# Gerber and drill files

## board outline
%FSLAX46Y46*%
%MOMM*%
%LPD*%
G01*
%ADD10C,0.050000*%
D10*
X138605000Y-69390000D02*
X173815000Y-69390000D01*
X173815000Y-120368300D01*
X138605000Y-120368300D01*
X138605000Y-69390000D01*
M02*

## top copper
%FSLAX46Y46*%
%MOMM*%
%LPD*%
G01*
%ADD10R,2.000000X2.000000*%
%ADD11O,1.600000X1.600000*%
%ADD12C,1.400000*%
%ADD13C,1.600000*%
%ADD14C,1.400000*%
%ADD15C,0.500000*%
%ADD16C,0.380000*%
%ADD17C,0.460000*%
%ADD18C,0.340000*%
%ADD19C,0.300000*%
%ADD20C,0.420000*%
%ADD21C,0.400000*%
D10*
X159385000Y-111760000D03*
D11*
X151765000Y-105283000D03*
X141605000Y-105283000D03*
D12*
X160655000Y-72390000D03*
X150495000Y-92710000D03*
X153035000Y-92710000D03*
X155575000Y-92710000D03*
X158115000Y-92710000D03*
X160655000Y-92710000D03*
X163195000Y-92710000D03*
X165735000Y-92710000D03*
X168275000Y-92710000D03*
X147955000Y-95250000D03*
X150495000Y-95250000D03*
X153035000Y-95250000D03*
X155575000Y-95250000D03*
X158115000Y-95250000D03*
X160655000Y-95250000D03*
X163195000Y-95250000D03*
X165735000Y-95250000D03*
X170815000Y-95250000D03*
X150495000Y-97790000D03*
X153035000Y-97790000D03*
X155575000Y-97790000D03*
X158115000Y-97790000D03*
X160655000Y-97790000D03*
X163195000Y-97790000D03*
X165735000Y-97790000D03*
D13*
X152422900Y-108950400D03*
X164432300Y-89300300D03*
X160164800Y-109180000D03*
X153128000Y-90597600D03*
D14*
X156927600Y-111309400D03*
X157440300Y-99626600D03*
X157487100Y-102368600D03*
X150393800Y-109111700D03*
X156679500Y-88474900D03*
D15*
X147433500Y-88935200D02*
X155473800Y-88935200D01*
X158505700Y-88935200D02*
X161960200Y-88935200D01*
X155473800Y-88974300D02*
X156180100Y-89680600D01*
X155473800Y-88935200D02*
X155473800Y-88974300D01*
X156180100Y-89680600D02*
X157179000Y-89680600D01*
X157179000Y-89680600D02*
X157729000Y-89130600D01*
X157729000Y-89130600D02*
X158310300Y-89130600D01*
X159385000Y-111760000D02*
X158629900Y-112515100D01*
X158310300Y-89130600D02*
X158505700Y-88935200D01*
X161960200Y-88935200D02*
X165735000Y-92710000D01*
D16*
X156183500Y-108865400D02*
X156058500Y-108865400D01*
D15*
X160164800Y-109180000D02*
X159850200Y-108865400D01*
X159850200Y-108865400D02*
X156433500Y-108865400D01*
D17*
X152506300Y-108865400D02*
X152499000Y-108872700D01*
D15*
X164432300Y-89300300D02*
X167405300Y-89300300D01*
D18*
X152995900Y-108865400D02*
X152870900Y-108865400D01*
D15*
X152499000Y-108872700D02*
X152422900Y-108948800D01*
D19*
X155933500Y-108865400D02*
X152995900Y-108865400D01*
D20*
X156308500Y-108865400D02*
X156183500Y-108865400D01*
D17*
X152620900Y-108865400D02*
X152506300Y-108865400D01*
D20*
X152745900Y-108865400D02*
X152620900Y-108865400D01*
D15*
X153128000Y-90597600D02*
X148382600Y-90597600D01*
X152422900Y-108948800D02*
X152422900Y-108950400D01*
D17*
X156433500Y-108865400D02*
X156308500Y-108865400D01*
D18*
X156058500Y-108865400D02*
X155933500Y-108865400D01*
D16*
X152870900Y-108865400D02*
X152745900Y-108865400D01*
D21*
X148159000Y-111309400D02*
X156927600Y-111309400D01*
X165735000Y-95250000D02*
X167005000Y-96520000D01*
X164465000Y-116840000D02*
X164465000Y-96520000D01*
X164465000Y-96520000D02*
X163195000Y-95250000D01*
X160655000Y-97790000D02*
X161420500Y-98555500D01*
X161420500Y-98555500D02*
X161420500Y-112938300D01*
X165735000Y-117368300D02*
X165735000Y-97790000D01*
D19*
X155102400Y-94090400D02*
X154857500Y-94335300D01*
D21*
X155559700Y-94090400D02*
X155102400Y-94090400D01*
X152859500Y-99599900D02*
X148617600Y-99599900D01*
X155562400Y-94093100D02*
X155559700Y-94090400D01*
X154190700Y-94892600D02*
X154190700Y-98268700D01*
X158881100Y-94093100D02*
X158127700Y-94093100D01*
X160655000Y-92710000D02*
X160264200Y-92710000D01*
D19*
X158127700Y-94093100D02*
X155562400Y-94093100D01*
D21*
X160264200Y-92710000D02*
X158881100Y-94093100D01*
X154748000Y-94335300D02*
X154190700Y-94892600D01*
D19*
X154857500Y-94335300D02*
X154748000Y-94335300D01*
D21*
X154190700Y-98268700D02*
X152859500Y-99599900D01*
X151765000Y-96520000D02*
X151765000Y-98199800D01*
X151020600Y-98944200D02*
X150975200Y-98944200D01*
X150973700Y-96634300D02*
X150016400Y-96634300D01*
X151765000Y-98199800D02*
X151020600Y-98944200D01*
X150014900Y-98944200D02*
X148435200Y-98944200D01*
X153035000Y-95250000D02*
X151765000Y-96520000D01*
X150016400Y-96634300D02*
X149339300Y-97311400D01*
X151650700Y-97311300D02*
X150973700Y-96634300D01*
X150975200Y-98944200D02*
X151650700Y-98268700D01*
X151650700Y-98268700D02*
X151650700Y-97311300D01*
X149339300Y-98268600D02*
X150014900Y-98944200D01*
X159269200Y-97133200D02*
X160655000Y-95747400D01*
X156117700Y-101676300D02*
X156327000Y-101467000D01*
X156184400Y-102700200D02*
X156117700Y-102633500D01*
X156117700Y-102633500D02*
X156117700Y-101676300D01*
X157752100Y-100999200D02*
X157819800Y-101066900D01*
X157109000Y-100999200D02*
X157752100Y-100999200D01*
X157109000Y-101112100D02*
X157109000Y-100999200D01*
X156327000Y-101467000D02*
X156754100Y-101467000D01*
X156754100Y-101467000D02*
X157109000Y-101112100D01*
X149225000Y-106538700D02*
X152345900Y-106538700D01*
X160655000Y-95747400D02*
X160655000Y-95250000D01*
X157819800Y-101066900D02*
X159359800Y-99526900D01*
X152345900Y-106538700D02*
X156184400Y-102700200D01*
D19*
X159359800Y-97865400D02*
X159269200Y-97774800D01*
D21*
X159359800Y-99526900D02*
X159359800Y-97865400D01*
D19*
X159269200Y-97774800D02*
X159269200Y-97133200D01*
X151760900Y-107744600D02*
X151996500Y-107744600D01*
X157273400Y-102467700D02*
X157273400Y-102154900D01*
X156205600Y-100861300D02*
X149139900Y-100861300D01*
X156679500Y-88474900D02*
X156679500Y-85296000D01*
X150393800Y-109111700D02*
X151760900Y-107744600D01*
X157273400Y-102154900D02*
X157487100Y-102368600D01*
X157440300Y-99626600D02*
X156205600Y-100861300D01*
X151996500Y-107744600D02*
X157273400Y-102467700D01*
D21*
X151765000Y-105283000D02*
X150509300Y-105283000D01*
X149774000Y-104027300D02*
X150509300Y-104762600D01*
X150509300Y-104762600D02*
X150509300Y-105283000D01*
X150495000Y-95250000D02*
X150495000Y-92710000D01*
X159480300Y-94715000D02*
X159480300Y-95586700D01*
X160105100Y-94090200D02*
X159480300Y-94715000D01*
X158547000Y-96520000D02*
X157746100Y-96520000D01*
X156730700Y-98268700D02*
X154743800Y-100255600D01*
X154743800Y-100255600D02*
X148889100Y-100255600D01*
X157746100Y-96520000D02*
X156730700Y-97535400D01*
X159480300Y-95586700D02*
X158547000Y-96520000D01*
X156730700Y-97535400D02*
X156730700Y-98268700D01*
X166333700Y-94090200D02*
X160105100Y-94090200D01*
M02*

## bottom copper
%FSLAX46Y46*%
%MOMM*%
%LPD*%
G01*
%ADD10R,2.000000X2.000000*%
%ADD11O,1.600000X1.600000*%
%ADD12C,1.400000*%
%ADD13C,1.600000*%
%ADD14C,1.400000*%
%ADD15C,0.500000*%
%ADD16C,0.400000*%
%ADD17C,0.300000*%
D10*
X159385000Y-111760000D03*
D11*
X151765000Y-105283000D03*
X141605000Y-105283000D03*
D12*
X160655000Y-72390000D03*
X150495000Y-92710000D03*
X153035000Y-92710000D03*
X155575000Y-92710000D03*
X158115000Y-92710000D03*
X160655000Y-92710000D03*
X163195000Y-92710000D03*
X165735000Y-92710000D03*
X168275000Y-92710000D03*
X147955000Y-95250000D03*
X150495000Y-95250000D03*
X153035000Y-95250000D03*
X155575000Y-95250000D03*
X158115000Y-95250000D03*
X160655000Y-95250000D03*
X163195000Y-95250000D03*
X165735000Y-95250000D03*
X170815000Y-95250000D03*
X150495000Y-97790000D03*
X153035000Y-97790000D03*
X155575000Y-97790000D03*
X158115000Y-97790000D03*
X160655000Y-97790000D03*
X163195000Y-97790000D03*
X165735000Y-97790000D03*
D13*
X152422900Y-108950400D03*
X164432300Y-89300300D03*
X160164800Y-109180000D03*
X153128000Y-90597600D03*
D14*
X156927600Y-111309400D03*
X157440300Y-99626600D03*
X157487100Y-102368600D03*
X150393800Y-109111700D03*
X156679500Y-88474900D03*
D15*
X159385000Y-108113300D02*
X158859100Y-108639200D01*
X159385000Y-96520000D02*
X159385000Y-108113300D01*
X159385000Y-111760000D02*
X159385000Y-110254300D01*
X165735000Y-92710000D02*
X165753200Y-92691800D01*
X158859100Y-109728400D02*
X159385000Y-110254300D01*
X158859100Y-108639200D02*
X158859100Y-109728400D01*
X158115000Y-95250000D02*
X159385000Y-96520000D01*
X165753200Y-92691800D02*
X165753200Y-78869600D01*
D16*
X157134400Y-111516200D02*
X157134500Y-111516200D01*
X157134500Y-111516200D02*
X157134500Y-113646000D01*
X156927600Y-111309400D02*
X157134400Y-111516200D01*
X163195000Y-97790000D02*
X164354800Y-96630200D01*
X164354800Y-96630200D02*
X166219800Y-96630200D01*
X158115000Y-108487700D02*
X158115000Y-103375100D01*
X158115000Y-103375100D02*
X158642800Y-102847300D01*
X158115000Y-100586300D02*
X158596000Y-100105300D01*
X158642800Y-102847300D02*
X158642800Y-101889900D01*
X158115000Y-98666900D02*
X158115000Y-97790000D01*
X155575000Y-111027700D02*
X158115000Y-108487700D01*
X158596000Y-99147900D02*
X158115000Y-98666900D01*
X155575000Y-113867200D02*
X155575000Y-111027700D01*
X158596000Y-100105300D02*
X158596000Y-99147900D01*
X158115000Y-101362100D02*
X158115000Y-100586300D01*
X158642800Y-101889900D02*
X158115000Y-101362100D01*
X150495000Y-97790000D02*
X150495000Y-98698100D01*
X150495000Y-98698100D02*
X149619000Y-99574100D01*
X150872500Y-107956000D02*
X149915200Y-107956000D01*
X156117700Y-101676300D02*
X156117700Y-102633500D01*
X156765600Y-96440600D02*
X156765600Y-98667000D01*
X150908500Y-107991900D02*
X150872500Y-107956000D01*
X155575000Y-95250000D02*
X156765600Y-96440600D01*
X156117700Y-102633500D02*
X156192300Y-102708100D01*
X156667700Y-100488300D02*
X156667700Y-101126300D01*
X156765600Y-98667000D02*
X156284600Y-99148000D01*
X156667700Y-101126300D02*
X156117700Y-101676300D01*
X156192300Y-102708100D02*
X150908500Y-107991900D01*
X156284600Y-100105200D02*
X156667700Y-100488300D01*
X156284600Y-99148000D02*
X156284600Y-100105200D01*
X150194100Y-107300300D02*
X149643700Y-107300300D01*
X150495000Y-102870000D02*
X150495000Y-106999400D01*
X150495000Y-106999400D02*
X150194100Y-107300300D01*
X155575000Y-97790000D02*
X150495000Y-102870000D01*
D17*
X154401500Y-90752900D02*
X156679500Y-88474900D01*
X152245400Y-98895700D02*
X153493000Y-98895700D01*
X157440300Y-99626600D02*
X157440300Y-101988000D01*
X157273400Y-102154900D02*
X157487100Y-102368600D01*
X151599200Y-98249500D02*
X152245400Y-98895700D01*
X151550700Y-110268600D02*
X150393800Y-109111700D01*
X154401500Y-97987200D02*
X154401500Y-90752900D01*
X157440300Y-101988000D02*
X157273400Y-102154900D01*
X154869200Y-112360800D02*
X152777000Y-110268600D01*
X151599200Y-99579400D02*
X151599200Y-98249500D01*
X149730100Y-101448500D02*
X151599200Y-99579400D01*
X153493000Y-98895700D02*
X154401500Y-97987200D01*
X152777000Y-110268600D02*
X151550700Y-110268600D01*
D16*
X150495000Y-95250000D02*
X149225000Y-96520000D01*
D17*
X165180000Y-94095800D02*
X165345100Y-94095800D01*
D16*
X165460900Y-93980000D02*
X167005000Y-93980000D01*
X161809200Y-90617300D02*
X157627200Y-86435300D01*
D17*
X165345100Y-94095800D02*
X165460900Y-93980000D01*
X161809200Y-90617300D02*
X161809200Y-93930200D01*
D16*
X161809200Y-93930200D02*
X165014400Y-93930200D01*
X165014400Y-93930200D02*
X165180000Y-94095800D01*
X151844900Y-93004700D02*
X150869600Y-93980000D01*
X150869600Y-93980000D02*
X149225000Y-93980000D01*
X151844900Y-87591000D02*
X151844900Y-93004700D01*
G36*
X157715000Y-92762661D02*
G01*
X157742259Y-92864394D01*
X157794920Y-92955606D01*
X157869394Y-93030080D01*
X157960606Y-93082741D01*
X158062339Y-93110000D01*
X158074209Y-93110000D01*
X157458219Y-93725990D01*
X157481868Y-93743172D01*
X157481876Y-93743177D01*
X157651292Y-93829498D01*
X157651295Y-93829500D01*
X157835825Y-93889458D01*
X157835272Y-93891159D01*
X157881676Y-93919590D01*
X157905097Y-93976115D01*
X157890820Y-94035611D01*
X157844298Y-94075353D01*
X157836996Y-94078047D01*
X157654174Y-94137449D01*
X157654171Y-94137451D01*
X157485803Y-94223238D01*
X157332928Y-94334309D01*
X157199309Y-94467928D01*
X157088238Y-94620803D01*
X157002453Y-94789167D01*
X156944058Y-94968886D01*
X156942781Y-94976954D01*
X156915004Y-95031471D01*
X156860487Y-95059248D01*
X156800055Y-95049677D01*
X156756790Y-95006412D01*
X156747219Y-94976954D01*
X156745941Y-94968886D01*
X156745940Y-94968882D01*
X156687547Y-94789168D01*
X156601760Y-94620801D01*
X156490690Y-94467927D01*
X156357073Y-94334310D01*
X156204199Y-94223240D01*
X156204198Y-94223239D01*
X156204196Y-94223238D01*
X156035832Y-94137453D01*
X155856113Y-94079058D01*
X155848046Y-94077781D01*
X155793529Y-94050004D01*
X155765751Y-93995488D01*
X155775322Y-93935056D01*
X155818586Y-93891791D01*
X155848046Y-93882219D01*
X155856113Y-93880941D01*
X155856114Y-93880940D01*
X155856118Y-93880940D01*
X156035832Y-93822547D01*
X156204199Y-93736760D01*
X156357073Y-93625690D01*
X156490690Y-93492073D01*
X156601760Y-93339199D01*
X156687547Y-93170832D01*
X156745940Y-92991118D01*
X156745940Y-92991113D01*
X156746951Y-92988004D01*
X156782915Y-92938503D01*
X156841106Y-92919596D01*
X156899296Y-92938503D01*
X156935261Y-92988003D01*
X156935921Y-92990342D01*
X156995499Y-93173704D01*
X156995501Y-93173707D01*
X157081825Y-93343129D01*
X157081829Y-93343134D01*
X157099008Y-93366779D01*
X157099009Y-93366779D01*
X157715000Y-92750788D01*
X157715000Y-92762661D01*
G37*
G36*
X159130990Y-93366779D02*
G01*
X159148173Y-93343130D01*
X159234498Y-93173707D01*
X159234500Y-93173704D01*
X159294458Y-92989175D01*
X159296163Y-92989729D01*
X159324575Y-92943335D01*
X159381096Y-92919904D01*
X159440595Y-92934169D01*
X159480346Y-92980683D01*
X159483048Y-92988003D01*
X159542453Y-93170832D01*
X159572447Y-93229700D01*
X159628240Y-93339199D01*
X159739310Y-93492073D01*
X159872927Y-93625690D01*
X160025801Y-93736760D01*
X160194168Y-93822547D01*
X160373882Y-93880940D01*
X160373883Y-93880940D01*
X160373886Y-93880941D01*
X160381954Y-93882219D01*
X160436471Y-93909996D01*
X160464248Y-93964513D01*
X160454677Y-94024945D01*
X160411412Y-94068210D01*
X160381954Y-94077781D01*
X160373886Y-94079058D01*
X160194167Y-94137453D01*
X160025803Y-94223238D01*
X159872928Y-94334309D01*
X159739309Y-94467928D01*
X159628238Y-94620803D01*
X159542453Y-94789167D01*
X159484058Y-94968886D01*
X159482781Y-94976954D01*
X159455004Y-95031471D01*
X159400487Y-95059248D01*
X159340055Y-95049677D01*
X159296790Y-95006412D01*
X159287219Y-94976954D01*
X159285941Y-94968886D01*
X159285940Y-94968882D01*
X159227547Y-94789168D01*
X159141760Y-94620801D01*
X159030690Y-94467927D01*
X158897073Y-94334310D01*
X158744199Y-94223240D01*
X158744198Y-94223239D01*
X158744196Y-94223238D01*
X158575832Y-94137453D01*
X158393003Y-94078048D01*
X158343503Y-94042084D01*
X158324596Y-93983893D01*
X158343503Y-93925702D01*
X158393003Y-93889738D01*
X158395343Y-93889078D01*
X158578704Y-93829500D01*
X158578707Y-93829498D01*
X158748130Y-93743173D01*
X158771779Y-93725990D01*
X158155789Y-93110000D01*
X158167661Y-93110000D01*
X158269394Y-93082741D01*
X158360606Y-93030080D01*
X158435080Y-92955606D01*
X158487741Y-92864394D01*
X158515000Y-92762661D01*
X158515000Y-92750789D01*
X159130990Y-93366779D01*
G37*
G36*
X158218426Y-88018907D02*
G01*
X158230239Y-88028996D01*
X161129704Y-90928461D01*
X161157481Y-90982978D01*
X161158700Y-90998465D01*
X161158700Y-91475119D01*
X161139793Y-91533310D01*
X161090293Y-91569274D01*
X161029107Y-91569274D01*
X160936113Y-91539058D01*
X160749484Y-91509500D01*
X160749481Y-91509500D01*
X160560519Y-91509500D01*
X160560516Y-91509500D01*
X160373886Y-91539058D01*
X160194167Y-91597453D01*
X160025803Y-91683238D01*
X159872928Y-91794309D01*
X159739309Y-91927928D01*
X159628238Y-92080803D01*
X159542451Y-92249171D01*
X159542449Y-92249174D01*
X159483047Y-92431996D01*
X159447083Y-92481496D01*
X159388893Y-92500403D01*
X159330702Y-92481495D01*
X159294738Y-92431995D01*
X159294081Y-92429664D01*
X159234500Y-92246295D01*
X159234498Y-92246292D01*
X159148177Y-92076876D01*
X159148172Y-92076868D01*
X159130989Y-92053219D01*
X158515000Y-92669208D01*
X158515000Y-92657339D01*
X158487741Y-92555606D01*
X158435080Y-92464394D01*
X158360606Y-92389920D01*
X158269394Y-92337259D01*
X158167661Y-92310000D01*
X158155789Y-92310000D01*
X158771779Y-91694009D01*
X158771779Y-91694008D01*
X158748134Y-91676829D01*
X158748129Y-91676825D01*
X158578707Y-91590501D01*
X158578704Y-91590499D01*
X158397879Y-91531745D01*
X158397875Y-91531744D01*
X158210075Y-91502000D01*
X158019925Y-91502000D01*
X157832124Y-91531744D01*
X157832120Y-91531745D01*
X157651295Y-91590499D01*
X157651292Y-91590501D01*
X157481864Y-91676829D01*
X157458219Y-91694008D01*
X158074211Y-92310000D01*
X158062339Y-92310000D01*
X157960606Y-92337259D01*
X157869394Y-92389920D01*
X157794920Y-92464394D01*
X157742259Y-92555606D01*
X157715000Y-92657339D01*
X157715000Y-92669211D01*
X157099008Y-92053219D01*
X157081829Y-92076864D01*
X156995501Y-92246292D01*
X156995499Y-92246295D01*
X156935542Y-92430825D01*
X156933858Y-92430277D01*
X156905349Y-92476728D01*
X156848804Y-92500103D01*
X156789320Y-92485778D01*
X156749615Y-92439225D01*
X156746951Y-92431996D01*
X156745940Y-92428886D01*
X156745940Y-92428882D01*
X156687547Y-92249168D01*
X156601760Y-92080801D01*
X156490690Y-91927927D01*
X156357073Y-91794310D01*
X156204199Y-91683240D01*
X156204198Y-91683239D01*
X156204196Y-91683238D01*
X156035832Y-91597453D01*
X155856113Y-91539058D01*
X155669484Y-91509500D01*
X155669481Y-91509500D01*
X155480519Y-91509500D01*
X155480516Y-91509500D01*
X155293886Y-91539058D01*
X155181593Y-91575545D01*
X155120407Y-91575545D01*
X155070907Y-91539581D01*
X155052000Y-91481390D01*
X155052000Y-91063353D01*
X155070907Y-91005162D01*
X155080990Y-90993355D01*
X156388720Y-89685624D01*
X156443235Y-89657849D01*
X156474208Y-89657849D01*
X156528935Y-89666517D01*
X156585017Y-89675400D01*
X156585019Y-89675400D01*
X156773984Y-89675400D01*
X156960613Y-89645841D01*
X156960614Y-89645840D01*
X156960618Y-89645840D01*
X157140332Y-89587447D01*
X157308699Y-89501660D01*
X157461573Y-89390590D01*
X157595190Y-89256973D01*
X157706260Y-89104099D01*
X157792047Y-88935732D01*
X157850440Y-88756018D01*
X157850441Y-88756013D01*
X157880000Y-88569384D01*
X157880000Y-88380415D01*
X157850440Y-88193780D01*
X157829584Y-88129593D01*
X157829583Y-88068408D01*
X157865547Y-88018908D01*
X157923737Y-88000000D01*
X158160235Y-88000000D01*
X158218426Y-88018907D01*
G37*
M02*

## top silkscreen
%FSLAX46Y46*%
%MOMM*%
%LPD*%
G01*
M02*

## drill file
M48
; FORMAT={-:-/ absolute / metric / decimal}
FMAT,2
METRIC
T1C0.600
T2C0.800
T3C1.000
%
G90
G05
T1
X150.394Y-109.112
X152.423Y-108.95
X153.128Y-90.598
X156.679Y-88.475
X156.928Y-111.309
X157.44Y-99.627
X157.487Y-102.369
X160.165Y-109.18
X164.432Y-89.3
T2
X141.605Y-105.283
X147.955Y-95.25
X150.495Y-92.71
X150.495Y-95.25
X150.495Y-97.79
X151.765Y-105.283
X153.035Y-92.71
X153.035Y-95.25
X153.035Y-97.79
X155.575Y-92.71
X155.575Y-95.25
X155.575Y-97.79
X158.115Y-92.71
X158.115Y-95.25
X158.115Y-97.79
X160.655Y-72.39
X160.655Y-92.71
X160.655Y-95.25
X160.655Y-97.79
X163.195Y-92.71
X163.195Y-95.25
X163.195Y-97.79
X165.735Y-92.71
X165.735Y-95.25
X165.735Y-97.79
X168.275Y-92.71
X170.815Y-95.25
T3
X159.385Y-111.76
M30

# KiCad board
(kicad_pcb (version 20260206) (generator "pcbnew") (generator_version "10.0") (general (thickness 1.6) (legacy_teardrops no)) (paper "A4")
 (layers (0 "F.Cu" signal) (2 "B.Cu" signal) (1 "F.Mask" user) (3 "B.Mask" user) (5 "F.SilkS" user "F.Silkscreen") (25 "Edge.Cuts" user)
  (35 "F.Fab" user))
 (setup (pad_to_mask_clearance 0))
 (gr_rect (start 138.605 69.39) (end 173.815 120.3683) (stroke (width 0.05) (type default)) (fill no) (layer "Edge.Cuts"))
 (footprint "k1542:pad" (layer "F.Cu") (at 159.385 111.76 0.0)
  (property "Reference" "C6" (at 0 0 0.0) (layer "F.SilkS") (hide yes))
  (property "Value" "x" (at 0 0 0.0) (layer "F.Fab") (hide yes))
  (pad "1" thru_hole rect (at 0 0 0.0) (size 2.0 2.0) (drill 1.0) (layers "*.Cu" "*.Mask") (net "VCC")))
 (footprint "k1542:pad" (layer "F.Cu") (at 151.765 105.283 90.0)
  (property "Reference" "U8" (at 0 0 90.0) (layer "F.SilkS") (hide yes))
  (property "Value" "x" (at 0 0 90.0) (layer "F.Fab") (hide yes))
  (pad "13" thru_hole oval (at 0 0 90.0) (size 1.6 1.6) (drill 0.8) (layers "*.Cu" "*.Mask") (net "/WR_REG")))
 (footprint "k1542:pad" (layer "F.Cu") (at 141.605 105.283 90.0)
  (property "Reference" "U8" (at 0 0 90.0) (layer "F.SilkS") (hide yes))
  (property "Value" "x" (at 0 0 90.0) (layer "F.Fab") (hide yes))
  (pad "17" thru_hole oval (at 0 0 90.0) (size 1.6 1.6) (drill 0.8) (layers "*.Cu" "*.Mask") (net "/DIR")))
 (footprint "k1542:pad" (layer "F.Cu") (at 160.655 72.39 180.0)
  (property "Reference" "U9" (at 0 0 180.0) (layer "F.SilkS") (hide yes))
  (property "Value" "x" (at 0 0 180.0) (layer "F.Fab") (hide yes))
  (pad "C8" thru_hole circle (at 0 0 180.0) (size 1.4 1.4) (drill 0.8) (layers "*.Cu" "*.Mask") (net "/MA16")))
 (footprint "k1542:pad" (layer "F.Cu") (at 150.495 92.71 180.0)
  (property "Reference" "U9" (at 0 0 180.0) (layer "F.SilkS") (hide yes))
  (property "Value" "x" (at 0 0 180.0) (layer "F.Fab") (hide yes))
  (pad "L4" thru_hole circle (at 0 0 180.0) (size 1.4 1.4) (drill 0.8) (layers "*.Cu" "*.Mask") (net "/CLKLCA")))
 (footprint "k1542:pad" (layer "F.Cu") (at 153.035 92.71 180.0)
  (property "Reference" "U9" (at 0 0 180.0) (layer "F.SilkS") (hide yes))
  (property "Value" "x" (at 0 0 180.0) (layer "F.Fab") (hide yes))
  (pad "L5" thru_hole circle (at 0 0 180.0) (size 1.4 1.4) (drill 0.8) (layers "*.Cu" "*.Mask") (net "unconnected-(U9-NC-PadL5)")))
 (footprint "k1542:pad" (layer "F.Cu") (at 155.575 92.71 180.0)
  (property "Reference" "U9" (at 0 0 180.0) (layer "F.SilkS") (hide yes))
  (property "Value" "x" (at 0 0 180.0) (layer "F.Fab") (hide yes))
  (pad "L6" thru_hole circle (at 0 0 180.0) (size 1.4 1.4) (drill 0.8) (layers "*.Cu" "*.Mask") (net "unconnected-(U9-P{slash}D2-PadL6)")))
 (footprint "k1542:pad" (layer "F.Cu") (at 158.115 92.71 180.0)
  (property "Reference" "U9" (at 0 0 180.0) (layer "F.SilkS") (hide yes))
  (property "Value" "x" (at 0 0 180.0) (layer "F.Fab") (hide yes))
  (pad "L7" thru_hole circle (at 0 0 180.0) (size 1.4 1.4) (drill 0.8) (layers "*.Cu" "*.Mask") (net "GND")))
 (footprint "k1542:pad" (layer "F.Cu") (at 160.655 92.71 180.0)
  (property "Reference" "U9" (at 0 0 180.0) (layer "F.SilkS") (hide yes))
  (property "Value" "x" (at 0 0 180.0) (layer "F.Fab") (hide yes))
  (pad "L8" thru_hole circle (at 0 0 180.0) (size 1.4 1.4) (drill 0.8) (layers "*.Cu" "*.Mask") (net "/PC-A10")))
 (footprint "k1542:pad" (layer "F.Cu") (at 163.195 92.71 180.0)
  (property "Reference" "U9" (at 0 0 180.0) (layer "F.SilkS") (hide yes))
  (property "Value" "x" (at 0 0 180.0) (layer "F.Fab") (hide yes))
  (pad "L9" thru_hole circle (at 0 0 180.0) (size 1.4 1.4) (drill 0.8) (layers "*.Cu" "*.Mask") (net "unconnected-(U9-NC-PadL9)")))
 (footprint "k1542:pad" (layer "F.Cu") (at 165.735 92.71 180.0)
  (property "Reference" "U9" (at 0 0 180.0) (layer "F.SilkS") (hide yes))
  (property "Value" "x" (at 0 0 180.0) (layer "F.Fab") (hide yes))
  (pad "L10" thru_hole circle (at 0 0 180.0) (size 1.4 1.4) (drill 0.8) (layers "*.Cu" "*.Mask") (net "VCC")))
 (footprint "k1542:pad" (layer "F.Cu") (at 168.275 92.71 180.0)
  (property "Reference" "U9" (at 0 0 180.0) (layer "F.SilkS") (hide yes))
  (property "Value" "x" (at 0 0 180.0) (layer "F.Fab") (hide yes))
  (pad "L11" thru_hole circle (at 0 0 180.0) (size 1.4 1.4) (drill 0.8) (layers "*.Cu" "*.Mask") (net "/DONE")))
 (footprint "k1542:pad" (layer "F.Cu") (at 147.955 95.25 180.0)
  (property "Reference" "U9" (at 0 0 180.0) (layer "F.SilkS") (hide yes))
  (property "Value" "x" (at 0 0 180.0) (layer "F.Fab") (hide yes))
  (pad "M3" thru_hole circle (at 0 0 180.0) (size 1.4 1.4) (drill 0.8) (layers "*.Cu" "*.Mask") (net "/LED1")))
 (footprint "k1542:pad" (layer "F.Cu") (at 150.495 95.25 180.0)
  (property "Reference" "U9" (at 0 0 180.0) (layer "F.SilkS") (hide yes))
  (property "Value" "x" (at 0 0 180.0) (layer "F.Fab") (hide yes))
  (pad "M4" thru_hole circle (at 0 0 180.0) (size 1.4 1.4) (drill 0.8) (layers "*.Cu" "*.Mask") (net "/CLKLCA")))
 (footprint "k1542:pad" (layer "F.Cu") (at 153.035 95.25 180.0)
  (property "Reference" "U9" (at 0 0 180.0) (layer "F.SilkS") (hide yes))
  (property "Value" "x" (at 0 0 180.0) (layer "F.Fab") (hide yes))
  (pad "M5" thru_hole circle (at 0 0 180.0) (size 1.4 1.4) (drill 0.8) (layers "*.Cu" "*.Mask") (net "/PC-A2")))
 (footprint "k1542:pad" (layer "F.Cu") (at 155.575 95.25 180.0)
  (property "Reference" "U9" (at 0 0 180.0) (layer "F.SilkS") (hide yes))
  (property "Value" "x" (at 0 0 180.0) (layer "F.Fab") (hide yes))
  (pad "M6" thru_hole circle (at 0 0 180.0) (size 1.4 1.4) (drill 0.8) (layers "*.Cu" "*.Mask") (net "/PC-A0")))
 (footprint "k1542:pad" (layer "F.Cu") (at 158.115 95.25 180.0)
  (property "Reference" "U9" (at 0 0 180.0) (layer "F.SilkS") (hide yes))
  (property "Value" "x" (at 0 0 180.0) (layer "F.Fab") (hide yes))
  (pad "M7" thru_hole circle (at 0 0 180.0) (size 1.4 1.4) (drill 0.8) (layers "*.Cu" "*.Mask") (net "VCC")))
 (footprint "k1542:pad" (layer "F.Cu") (at 160.655 95.25 180.0)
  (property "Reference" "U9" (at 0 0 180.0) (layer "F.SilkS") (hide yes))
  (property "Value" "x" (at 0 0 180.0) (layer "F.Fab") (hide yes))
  (pad "M8" thru_hole circle (at 0 0 180.0) (size 1.4 1.4) (drill 0.8) (layers "*.Cu" "*.Mask") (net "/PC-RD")))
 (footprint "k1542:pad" (layer "F.Cu") (at 163.195 95.25 180.0)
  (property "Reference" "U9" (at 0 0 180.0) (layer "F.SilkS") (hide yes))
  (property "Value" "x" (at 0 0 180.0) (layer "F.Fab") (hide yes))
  (pad "M9" thru_hole circle (at 0 0 180.0) (size 1.4 1.4) (drill 0.8) (layers "*.Cu" "*.Mask") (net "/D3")))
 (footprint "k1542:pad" (layer "F.Cu") (at 165.735 95.25 180.0)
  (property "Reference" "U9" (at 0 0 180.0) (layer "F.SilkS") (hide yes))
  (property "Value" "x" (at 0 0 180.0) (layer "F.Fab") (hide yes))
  (pad "M10" thru_hole circle (at 0 0 180.0) (size 1.4 1.4) (drill 0.8) (layers "*.Cu" "*.Mask") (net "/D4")))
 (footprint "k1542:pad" (layer "F.Cu") (at 170.815 95.25 180.0)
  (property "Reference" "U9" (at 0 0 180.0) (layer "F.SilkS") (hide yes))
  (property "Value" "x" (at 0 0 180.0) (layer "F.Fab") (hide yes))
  (pad "M12" thru_hole circle (at 0 0 180.0) (size 1.4 1.4) (drill 0.8) (layers "*.Cu" "*.Mask") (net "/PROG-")))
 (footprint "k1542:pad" (layer "F.Cu") (at 150.495 97.79 180.0)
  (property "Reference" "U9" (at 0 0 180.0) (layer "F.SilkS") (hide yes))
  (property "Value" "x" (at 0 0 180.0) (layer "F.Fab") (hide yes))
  (pad "N4" thru_hole circle (at 0 0 180.0) (size 1.4 1.4) (drill 0.8) (layers "*.Cu" "*.Mask") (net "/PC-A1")))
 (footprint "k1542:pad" (layer "F.Cu") (at 153.035 97.79 180.0)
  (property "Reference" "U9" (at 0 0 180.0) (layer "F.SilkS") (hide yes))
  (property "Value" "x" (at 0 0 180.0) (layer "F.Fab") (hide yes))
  (pad "N5" thru_hole circle (at 0 0 180.0) (size 1.4 1.4) (drill 0.8) (layers "*.Cu" "*.Mask") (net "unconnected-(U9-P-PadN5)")))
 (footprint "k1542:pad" (layer "F.Cu") (at 155.575 97.79 180.0)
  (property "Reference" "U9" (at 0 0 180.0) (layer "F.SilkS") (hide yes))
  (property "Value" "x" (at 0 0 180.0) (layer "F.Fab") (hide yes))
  (pad "N6" thru_hole circle (at 0 0 180.0) (size 1.4 1.4) (drill 0.8) (layers "*.Cu" "*.Mask") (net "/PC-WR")))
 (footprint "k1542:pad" (layer "F.Cu") (at 158.115 97.79 180.0)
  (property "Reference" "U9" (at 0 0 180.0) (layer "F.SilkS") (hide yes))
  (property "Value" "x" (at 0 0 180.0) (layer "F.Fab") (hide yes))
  (pad "N7" thru_hole circle (at 0 0 180.0) (size 1.4 1.4) (drill 0.8) (layers "*.Cu" "*.Mask") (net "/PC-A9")))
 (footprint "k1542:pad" (layer "F.Cu") (at 160.655 97.79 180.0)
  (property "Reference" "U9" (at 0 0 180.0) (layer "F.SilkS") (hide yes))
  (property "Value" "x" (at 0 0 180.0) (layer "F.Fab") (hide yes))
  (pad "N8" thru_hole circle (at 0 0 180.0) (size 1.4 1.4) (drill 0.8) (layers "*.Cu" "*.Mask") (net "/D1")))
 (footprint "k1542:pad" (layer "F.Cu") (at 163.195 97.79 180.0)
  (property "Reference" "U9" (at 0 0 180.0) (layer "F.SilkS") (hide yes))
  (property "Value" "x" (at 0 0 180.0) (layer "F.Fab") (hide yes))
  (pad "N9" thru_hole circle (at 0 0 180.0) (size 1.4 1.4) (drill 0.8) (layers "*.Cu" "*.Mask") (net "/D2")))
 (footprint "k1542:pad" (layer "F.Cu") (at 165.735 97.79 180.0)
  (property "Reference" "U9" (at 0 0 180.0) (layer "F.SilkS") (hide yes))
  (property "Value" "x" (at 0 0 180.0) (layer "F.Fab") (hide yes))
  (pad "N10" thru_hole circle (at 0 0 180.0) (size 1.4 1.4) (drill 0.8) (layers "*.Cu" "*.Mask") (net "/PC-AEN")))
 (via (at 152.4229 108.9504) (size 1.6) (drill 0.6) (layers "F.Cu" "B.Cu") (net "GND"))
 (via (at 164.4323 89.3003) (size 1.6) (drill 0.6) (layers "F.Cu" "B.Cu") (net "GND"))
 (via (at 160.1648 109.18) (size 1.6) (drill 0.6) (layers "F.Cu" "B.Cu") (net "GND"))
 (via (at 153.128 90.5976) (size 1.6) (drill 0.6) (layers "F.Cu" "B.Cu") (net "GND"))
 (via (at 156.9276 111.3094) (size 1.4) (drill 0.6) (layers "F.Cu" "B.Cu") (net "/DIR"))
 (via (at 157.4403 99.6266) (size 1.4) (drill 0.6) (layers "F.Cu" "B.Cu") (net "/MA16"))
 (via (at 157.4871 102.3686) (size 1.4) (drill 0.6) (layers "F.Cu" "B.Cu") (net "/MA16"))
 (via (at 150.3938 109.1117) (size 1.4) (drill 0.6) (layers "F.Cu" "B.Cu") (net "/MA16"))
 (via (at 156.6795 88.4749) (size 1.4) (drill 0.6) (layers "F.Cu" "B.Cu") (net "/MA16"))
 (segment (start 147.4335 88.9352) (end 155.4738 88.9352) (width 0.5) (layer "F.Cu") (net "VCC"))
 (segment (start 158.5057 88.9352) (end 161.9602 88.9352) (width 0.5) (layer "F.Cu") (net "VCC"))
 (segment (start 155.4738 88.9743) (end 156.1801 89.6806) (width 0.5) (layer "F.Cu") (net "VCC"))
 (segment (start 155.4738 88.9352) (end 155.4738 88.9743) (width 0.5) (layer "F.Cu") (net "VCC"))
 (segment (start 156.1801 89.6806) (end 157.179 89.6806) (width 0.5) (layer "F.Cu") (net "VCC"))
 (segment (start 157.179 89.6806) (end 157.729 89.1306) (width 0.5) (layer "F.Cu") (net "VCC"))
 (segment (start 157.729 89.1306) (end 158.3103 89.1306) (width 0.5) (layer "F.Cu") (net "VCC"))
 (segment (start 159.385 111.76) (end 158.6299 112.5151) (width 0.5) (layer "F.Cu") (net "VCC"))
 (segment (start 158.3103 89.1306) (end 158.5057 88.9352) (width 0.5) (layer "F.Cu") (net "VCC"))
 (segment (start 161.9602 88.9352) (end 165.735 92.71) (width 0.5) (layer "F.Cu") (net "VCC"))
 (segment (start 159.385 108.1133) (end 158.8591 108.6392) (width 0.5) (layer "B.Cu") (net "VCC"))
 (segment (start 159.385 96.52) (end 159.385 108.1133) (width 0.5) (layer "B.Cu") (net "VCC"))
 (segment (start 159.385 111.76) (end 159.385 110.2543) (width 0.5) (layer "B.Cu") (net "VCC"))
 (segment (start 165.735 92.71) (end 165.7532 92.6918) (width 0.5) (layer "B.Cu") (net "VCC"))
 (segment (start 158.8591 109.7284) (end 159.385 110.2543) (width 0.5) (layer "B.Cu") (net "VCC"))
 (segment (start 158.8591 108.6392) (end 158.8591 109.7284) (width 0.5) (layer "B.Cu") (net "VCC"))
 (segment (start 158.115 95.25) (end 159.385 96.52) (width 0.5) (layer "B.Cu") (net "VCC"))
 (segment (start 165.7532 92.6918) (end 165.7532 78.8696) (width 0.5) (layer "B.Cu") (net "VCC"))
 (segment (start 156.1835 108.8654) (end 156.0585 108.8654) (width 0.38) (layer "F.Cu") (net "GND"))
 (segment (start 160.1648 109.18) (end 159.8502 108.8654) (width 0.5) (layer "F.Cu") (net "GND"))
 (segment (start 159.8502 108.8654) (end 156.4335 108.8654) (width 0.5) (layer "F.Cu") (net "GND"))
 (segment (start 152.5063 108.8654) (end 152.499 108.8727) (width 0.46) (layer "F.Cu") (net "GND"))
 (segment (start 164.4323 89.3003) (end 167.4053 89.3003) (width 0.5) (layer "F.Cu") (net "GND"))
 (segment (start 152.9959 108.8654) (end 152.8709 108.8654) (width 0.34) (layer "F.Cu") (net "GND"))
 (segment (start 152.499 108.8727) (end 152.4229 108.9488) (width 0.5) (layer "F.Cu") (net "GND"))
 (segment (start 155.9335 108.8654) (end 152.9959 108.8654) (width 0.3) (layer "F.Cu") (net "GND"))
 (segment (start 156.3085 108.8654) (end 156.1835 108.8654) (width 0.42) (layer "F.Cu") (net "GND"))
 (segment (start 152.6209 108.8654) (end 152.5063 108.8654) (width 0.46) (layer "F.Cu") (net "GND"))
 (segment (start 152.7459 108.8654) (end 152.6209 108.8654) (width 0.42) (layer "F.Cu") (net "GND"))
 (segment (start 153.128 90.5976) (end 148.3826 90.5976) (width 0.5) (layer "F.Cu") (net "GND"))
 (segment (start 152.4229 108.9488) (end 152.4229 108.9504) (width 0.5) (layer "F.Cu") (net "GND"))
 (segment (start 156.4335 108.8654) (end 156.3085 108.8654) (width 0.46) (layer "F.Cu") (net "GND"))
 (segment (start 156.0585 108.8654) (end 155.9335 108.8654) (width 0.34) (layer "F.Cu") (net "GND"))
 (segment (start 152.8709 108.8654) (end 152.7459 108.8654) (width 0.38) (layer "F.Cu") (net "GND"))
 (segment (start 148.159 111.3094) (end 156.9276 111.3094) (width 0.4) (layer "F.Cu") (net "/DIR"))
 (segment (start 157.1344 111.5162) (end 157.1345 111.5162) (width 0.4) (layer "B.Cu") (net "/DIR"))
 (segment (start 157.1345 111.5162) (end 157.1345 113.646) (width 0.4) (layer "B.Cu") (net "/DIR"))
 (segment (start 156.9276 111.3094) (end 157.1344 111.5162) (width 0.4) (layer "B.Cu") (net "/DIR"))
 (segment (start 165.735 95.25) (end 167.005 96.52) (width 0.4) (layer "F.Cu") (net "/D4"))
 (segment (start 164.465 116.84) (end 164.465 96.52) (width 0.4) (layer "F.Cu") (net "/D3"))
 (segment (start 164.465 96.52) (end 163.195 95.25) (width 0.4) (layer "F.Cu") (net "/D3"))
 (segment (start 163.195 97.79) (end 164.3548 96.6302) (width 0.4) (layer "B.Cu") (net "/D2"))
 (segment (start 164.3548 96.6302) (end 166.2198 96.6302) (width 0.4) (layer "B.Cu") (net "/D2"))
 (segment (start 160.655 97.79) (end 161.4205 98.5555) (width 0.4) (layer "F.Cu") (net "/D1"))
 (segment (start 161.4205 98.5555) (end 161.4205 112.9383) (width 0.4) (layer "F.Cu") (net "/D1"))
 (segment (start 165.735 117.3683) (end 165.735 97.79) (width 0.4) (layer "F.Cu") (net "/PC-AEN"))
 (segment (start 158.115 108.4877) (end 158.115 103.3751) (width 0.4) (layer "B.Cu") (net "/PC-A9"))
 (segment (start 158.115 103.3751) (end 158.6428 102.8473) (width 0.4) (layer "B.Cu") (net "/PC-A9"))
 (segment (start 158.115 100.5863) (end 158.596 100.1053) (width 0.4) (layer "B.Cu") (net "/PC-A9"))
 (segment (start 158.6428 102.8473) (end 158.6428 101.8899) (width 0.4) (layer "B.Cu") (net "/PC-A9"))
 (segment (start 158.115 98.6669) (end 158.115 97.79) (width 0.4) (layer "B.Cu") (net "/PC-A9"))
 (segment (start 155.575 111.0277) (end 158.115 108.4877) (width 0.4) (layer "B.Cu") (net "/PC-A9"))
 (segment (start 158.596 99.1479) (end 158.115 98.6669) (width 0.4) (layer "B.Cu") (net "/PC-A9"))
 (segment (start 155.575 113.8672) (end 155.575 111.0277) (width 0.4) (layer "B.Cu") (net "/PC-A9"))
 (segment (start 158.596 100.1053) (end 158.596 99.1479) (width 0.4) (layer "B.Cu") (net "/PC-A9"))
 (segment (start 158.115 101.3621) (end 158.115 100.5863) (width 0.4) (layer "B.Cu") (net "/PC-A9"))
 (segment (start 158.6428 101.8899) (end 158.115 101.3621) (width 0.4) (layer "B.Cu") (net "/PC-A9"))
 (segment (start 155.1024 94.0904) (end 154.8575 94.3353) (width 0.3) (layer "F.Cu") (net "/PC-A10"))
 (segment (start 155.5597 94.0904) (end 155.1024 94.0904) (width 0.4) (layer "F.Cu") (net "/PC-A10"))
 (segment (start 152.8595 99.5999) (end 148.6176 99.5999) (width 0.4) (layer "F.Cu") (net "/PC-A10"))
 (segment (start 155.5624 94.0931) (end 155.5597 94.0904) (width 0.4) (layer "F.Cu") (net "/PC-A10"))
 (segment (start 154.1907 94.8926) (end 154.1907 98.2687) (width 0.4) (layer "F.Cu") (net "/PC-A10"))
 (segment (start 158.8811 94.0931) (end 158.1277 94.0931) (width 0.4) (layer "F.Cu") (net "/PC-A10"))
 (segment (start 160.655 92.71) (end 160.2642 92.71) (width 0.4) (layer "F.Cu") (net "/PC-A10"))
 (segment (start 158.1277 94.0931) (end 155.5624 94.0931) (width 0.3) (layer "F.Cu") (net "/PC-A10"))
 (segment (start 160.2642 92.71) (end 158.8811 94.0931) (width 0.4) (layer "F.Cu") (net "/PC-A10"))
 (segment (start 154.748 94.3353) (end 154.1907 94.8926) (width 0.4) (layer "F.Cu") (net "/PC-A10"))
 (segment (start 154.8575 94.3353) (end 154.748 94.3353) (width 0.3) (layer "F.Cu") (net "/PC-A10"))
 (segment (start 154.1907 98.2687) (end 152.8595 99.5999) (width 0.4) (layer "F.Cu") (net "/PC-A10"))
 (segment (start 150.495 97.79) (end 150.495 98.6981) (width 0.4) (layer "B.Cu") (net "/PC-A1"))
 (segment (start 150.495 98.6981) (end 149.619 99.5741) (width 0.4) (layer "B.Cu") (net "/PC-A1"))
 (segment (start 150.8725 107.956) (end 149.9152 107.956) (width 0.4) (layer "B.Cu") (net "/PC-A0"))
 (segment (start 156.1177 101.6763) (end 156.1177 102.6335) (width 0.4) (layer "B.Cu") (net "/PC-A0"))
 (segment (start 156.7656 96.4406) (end 156.7656 98.667) (width 0.4) (layer "B.Cu") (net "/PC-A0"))
 (segment (start 150.9085 107.9919) (end 150.8725 107.956) (width 0.4) (layer "B.Cu") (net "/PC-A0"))
 (segment (start 155.575 95.25) (end 156.7656 96.4406) (width 0.4) (layer "B.Cu") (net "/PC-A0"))
 (segment (start 156.1177 102.6335) (end 156.1923 102.7081) (width 0.4) (layer "B.Cu") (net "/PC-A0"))
 (segment (start 156.6677 100.4883) (end 156.6677 101.1263) (width 0.4) (layer "B.Cu") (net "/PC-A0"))
 (segment (start 156.7656 98.667) (end 156.2846 99.148) (width 0.4) (layer "B.Cu") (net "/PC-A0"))
 (segment (start 156.6677 101.1263) (end 156.1177 101.6763) (width 0.4) (layer "B.Cu") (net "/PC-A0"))
 (segment (start 156.1923 102.7081) (end 150.9085 107.9919) (width 0.4) (layer "B.Cu") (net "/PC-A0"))
 (segment (start 156.2846 100.1052) (end 156.6677 100.4883) (width 0.4) (layer "B.Cu") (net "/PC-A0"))
 (segment (start 156.2846 99.148) (end 156.2846 100.1052) (width 0.4) (layer "B.Cu") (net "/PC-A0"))
 (segment (start 151.765 96.52) (end 151.765 98.1998) (width 0.4) (layer "F.Cu") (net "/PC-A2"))
 (segment (start 151.0206 98.9442) (end 150.9752 98.9442) (width 0.4) (layer "F.Cu") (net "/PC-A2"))
 (segment (start 150.9737 96.6343) (end 150.0164 96.6343) (width 0.4) (layer "F.Cu") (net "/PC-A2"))
 (segment (start 151.765 98.1998) (end 151.0206 98.9442) (width 0.4) (layer "F.Cu") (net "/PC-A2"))
 (segment (start 150.0149 98.9442) (end 148.4352 98.9442) (width 0.4) (layer "F.Cu") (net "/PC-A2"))
 (segment (start 153.035 95.25) (end 151.765 96.52) (width 0.4) (layer "F.Cu") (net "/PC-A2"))
 (segment (start 150.0164 96.6343) (end 149.3393 97.3114) (width 0.4) (layer "F.Cu") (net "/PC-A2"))
 (segment (start 151.6507 97.3113) (end 150.9737 96.6343) (width 0.4) (layer "F.Cu") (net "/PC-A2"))
 (segment (start 150.9752 98.9442) (end 151.6507 98.2687) (width 0.4) (layer "F.Cu") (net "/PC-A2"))
 (segment (start 151.6507 98.2687) (end 151.6507 97.3113) (width 0.4) (layer "F.Cu") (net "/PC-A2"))
 (segment (start 149.3393 98.2686) (end 150.0149 98.9442) (width 0.4) (layer "F.Cu") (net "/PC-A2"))
 (segment (start 159.2692 97.1332) (end 160.655 95.7474) (width 0.4) (layer "F.Cu") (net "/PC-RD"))
 (segment (start 156.1177 101.6763) (end 156.327 101.467) (width 0.4) (layer "F.Cu") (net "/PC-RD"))
 (segment (start 156.1844 102.7002) (end 156.1177 102.6335) (width 0.4) (layer "F.Cu") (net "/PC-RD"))
 (segment (start 156.1177 102.6335) (end 156.1177 101.6763) (width 0.4) (layer "F.Cu") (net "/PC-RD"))
 (segment (start 157.7521 100.9992) (end 157.8198 101.0669) (width 0.4) (layer "F.Cu") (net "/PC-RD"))
 (segment (start 157.109 100.9992) (end 157.7521 100.9992) (width 0.4) (layer "F.Cu") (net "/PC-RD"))
 (segment (start 157.109 101.1121) (end 157.109 100.9992) (width 0.4) (layer "F.Cu") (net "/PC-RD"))
 (segment (start 156.327 101.467) (end 156.7541 101.467) (width 0.4) (layer "F.Cu") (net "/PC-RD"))
 (segment (start 156.7541 101.467) (end 157.109 101.1121) (width 0.4) (layer "F.Cu") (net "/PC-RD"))
 (segment (start 149.225 106.5387) (end 152.3459 106.5387) (width 0.4) (layer "F.Cu") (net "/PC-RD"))
 (segment (start 160.655 95.7474) (end 160.655 95.25) (width 0.4) (layer "F.Cu") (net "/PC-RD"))
 (segment (start 157.8198 101.0669) (end 159.3598 99.5269) (width 0.4) (layer "F.Cu") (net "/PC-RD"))
 (segment (start 152.3459 106.5387) (end 156.1844 102.7002) (width 0.4) (layer "F.Cu") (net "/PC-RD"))
 (segment (start 159.3598 97.8654) (end 159.2692 97.7748) (width 0.3) (layer "F.Cu") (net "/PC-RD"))
 (segment (start 159.3598 99.5269) (end 159.3598 97.8654) (width 0.4) (layer "F.Cu") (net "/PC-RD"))
 (segment (start 159.2692 97.7748) (end 159.2692 97.1332) (width 0.3) (layer "F.Cu") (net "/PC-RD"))
 (segment (start 150.1941 107.3003) (end 149.6437 107.3003) (width 0.4) (layer "B.Cu") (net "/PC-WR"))
 (segment (start 150.495 102.87) (end 150.495 106.9994) (width 0.4) (layer "B.Cu") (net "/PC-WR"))
 (segment (start 150.495 106.9994) (end 150.1941 107.3003) (width 0.4) (layer "B.Cu") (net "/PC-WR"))
 (segment (start 155.575 97.79) (end 150.495 102.87) (width 0.4) (layer "B.Cu") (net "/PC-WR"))
 (segment (start 151.7609 107.7446) (end 151.9965 107.7446) (width 0.3) (layer "F.Cu") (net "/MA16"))
 (segment (start 157.2734 102.4677) (end 157.2734 102.1549) (width 0.3) (layer "F.Cu") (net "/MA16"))
 (segment (start 156.2056 100.8613) (end 149.1399 100.8613) (width 0.3) (layer "F.Cu") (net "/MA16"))
 (segment (start 156.6795 88.4749) (end 156.6795 85.296) (width 0.3) (layer "F.Cu") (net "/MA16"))
 (segment (start 150.3938 109.1117) (end 151.7609 107.7446) (width 0.3) (layer "F.Cu") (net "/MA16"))
 (segment (start 157.2734 102.1549) (end 157.4871 102.3686) (width 0.3) (layer "F.Cu") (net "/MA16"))
 (segment (start 157.4403 99.6266) (end 156.2056 100.8613) (width 0.3) (layer "F.Cu") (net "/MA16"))
 (segment (start 151.9965 107.7446) (end 157.2734 102.4677) (width 0.3) (layer "F.Cu") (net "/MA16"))
 (segment (start 154.4015 90.7529) (end 156.6795 88.4749) (width 0.3) (layer "B.Cu") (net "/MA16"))
 (segment (start 152.2454 98.8957) (end 153.493 98.8957) (width 0.3) (layer "B.Cu") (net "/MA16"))
 (segment (start 157.4403 99.6266) (end 157.4403 101.988) (width 0.3) (layer "B.Cu") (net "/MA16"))
 (segment (start 157.2734 102.1549) (end 157.4871 102.3686) (width 0.3) (layer "B.Cu") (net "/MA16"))
 (segment (start 151.5992 98.2495) (end 152.2454 98.8957) (width 0.3) (layer "B.Cu") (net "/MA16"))
 (segment (start 151.5507 110.2686) (end 150.3938 109.1117) (width 0.3) (layer "B.Cu") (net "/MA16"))
 (segment (start 154.4015 97.9872) (end 154.4015 90.7529) (width 0.3) (layer "B.Cu") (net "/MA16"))
 (segment (start 157.4403 101.988) (end 157.2734 102.1549) (width 0.3) (layer "B.Cu") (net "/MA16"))
 (segment (start 154.8692 112.3608) (end 152.777 110.2686) (width 0.3) (layer "B.Cu") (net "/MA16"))
 (segment (start 151.5992 99.5794) (end 151.5992 98.2495) (width 0.3) (layer "B.Cu") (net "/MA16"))
 (segment (start 149.7301 101.4485) (end 151.5992 99.5794) (width 0.3) (layer "B.Cu") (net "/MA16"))
 (segment (start 153.493 98.8957) (end 154.4015 97.9872) (width 0.3) (layer "B.Cu") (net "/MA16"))
 (segment (start 152.777 110.2686) (end 151.5507 110.2686) (width 0.3) (layer "B.Cu") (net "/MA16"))
 (segment (start 151.765 105.283) (end 150.5093 105.283) (width 0.4) (layer "F.Cu") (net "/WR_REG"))
 (segment (start 149.774 104.0273) (end 150.5093 104.7626) (width 0.4) (layer "F.Cu") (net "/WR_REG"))
 (segment (start 150.5093 104.7626) (end 150.5093 105.283) (width 0.4) (layer "F.Cu") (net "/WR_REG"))
 (segment (start 150.495 95.25) (end 150.495 92.71) (width 0.4) (layer "F.Cu") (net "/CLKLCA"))
 (segment (start 150.495 95.25) (end 149.225 96.52) (width 0.4) (layer "B.Cu") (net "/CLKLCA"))
 (segment (start 159.4803 94.715) (end 159.4803 95.5867) (width 0.4) (layer "F.Cu") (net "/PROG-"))
 (segment (start 160.1051 94.0902) (end 159.4803 94.715) (width 0.4) (layer "F.Cu") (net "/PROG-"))
 (segment (start 158.547 96.52) (end 157.7461 96.52) (width 0.4) (layer "F.Cu") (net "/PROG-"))
 (segment (start 156.7307 98.2687) (end 154.7438 100.2556) (width 0.4) (layer "F.Cu") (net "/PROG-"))
 (segment (start 154.7438 100.2556) (end 148.8891 100.2556) (width 0.4) (layer "F.Cu") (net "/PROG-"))
 (segment (start 157.7461 96.52) (end 156.7307 97.5354) (width 0.4) (layer "F.Cu") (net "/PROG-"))
 (segment (start 159.4803 95.5867) (end 158.547 96.52) (width 0.4) (layer "F.Cu") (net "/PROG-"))
 (segment (start 156.7307 97.5354) (end 156.7307 98.2687) (width 0.4) (layer "F.Cu") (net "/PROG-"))
 (segment (start 166.3337 94.0902) (end 160.1051 94.0902) (width 0.4) (layer "F.Cu") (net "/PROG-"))
 (segment (start 165.18 94.0958) (end 165.3451 94.0958) (width 0.3) (layer "B.Cu") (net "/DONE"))
 (segment (start 165.4609 93.98) (end 167.005 93.98) (width 0.4) (layer "B.Cu") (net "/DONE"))
 (segment (start 161.8092 90.6173) (end 157.6272 86.4353) (width 0.4) (layer "B.Cu") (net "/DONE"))
 (segment (start 165.3451 94.0958) (end 165.4609 93.98) (width 0.3) (layer "B.Cu") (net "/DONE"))
 (segment (start 161.8092 90.6173) (end 161.8092 93.9302) (width 0.3) (layer "B.Cu") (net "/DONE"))
 (segment (start 161.8092 93.9302) (end 165.0144 93.9302) (width 0.4) (layer "B.Cu") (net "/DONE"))
 (segment (start 165.0144 93.9302) (end 165.18 94.0958) (width 0.4) (layer "B.Cu") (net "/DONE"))
 (segment (start 151.8449 93.0047) (end 150.8696 93.98) (width 0.4) (layer "B.Cu") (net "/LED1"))
 (segment (start 150.8696 93.98) (end 149.225 93.98) (width 0.4) (layer "B.Cu") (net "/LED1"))
 (segment (start 151.8449 87.591) (end 151.8449 93.0047) (width 0.4) (layer "B.Cu") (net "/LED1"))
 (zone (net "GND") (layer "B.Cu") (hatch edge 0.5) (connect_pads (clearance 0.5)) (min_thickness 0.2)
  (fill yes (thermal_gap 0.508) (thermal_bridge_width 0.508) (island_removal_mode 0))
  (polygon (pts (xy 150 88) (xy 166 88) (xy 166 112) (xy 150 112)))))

